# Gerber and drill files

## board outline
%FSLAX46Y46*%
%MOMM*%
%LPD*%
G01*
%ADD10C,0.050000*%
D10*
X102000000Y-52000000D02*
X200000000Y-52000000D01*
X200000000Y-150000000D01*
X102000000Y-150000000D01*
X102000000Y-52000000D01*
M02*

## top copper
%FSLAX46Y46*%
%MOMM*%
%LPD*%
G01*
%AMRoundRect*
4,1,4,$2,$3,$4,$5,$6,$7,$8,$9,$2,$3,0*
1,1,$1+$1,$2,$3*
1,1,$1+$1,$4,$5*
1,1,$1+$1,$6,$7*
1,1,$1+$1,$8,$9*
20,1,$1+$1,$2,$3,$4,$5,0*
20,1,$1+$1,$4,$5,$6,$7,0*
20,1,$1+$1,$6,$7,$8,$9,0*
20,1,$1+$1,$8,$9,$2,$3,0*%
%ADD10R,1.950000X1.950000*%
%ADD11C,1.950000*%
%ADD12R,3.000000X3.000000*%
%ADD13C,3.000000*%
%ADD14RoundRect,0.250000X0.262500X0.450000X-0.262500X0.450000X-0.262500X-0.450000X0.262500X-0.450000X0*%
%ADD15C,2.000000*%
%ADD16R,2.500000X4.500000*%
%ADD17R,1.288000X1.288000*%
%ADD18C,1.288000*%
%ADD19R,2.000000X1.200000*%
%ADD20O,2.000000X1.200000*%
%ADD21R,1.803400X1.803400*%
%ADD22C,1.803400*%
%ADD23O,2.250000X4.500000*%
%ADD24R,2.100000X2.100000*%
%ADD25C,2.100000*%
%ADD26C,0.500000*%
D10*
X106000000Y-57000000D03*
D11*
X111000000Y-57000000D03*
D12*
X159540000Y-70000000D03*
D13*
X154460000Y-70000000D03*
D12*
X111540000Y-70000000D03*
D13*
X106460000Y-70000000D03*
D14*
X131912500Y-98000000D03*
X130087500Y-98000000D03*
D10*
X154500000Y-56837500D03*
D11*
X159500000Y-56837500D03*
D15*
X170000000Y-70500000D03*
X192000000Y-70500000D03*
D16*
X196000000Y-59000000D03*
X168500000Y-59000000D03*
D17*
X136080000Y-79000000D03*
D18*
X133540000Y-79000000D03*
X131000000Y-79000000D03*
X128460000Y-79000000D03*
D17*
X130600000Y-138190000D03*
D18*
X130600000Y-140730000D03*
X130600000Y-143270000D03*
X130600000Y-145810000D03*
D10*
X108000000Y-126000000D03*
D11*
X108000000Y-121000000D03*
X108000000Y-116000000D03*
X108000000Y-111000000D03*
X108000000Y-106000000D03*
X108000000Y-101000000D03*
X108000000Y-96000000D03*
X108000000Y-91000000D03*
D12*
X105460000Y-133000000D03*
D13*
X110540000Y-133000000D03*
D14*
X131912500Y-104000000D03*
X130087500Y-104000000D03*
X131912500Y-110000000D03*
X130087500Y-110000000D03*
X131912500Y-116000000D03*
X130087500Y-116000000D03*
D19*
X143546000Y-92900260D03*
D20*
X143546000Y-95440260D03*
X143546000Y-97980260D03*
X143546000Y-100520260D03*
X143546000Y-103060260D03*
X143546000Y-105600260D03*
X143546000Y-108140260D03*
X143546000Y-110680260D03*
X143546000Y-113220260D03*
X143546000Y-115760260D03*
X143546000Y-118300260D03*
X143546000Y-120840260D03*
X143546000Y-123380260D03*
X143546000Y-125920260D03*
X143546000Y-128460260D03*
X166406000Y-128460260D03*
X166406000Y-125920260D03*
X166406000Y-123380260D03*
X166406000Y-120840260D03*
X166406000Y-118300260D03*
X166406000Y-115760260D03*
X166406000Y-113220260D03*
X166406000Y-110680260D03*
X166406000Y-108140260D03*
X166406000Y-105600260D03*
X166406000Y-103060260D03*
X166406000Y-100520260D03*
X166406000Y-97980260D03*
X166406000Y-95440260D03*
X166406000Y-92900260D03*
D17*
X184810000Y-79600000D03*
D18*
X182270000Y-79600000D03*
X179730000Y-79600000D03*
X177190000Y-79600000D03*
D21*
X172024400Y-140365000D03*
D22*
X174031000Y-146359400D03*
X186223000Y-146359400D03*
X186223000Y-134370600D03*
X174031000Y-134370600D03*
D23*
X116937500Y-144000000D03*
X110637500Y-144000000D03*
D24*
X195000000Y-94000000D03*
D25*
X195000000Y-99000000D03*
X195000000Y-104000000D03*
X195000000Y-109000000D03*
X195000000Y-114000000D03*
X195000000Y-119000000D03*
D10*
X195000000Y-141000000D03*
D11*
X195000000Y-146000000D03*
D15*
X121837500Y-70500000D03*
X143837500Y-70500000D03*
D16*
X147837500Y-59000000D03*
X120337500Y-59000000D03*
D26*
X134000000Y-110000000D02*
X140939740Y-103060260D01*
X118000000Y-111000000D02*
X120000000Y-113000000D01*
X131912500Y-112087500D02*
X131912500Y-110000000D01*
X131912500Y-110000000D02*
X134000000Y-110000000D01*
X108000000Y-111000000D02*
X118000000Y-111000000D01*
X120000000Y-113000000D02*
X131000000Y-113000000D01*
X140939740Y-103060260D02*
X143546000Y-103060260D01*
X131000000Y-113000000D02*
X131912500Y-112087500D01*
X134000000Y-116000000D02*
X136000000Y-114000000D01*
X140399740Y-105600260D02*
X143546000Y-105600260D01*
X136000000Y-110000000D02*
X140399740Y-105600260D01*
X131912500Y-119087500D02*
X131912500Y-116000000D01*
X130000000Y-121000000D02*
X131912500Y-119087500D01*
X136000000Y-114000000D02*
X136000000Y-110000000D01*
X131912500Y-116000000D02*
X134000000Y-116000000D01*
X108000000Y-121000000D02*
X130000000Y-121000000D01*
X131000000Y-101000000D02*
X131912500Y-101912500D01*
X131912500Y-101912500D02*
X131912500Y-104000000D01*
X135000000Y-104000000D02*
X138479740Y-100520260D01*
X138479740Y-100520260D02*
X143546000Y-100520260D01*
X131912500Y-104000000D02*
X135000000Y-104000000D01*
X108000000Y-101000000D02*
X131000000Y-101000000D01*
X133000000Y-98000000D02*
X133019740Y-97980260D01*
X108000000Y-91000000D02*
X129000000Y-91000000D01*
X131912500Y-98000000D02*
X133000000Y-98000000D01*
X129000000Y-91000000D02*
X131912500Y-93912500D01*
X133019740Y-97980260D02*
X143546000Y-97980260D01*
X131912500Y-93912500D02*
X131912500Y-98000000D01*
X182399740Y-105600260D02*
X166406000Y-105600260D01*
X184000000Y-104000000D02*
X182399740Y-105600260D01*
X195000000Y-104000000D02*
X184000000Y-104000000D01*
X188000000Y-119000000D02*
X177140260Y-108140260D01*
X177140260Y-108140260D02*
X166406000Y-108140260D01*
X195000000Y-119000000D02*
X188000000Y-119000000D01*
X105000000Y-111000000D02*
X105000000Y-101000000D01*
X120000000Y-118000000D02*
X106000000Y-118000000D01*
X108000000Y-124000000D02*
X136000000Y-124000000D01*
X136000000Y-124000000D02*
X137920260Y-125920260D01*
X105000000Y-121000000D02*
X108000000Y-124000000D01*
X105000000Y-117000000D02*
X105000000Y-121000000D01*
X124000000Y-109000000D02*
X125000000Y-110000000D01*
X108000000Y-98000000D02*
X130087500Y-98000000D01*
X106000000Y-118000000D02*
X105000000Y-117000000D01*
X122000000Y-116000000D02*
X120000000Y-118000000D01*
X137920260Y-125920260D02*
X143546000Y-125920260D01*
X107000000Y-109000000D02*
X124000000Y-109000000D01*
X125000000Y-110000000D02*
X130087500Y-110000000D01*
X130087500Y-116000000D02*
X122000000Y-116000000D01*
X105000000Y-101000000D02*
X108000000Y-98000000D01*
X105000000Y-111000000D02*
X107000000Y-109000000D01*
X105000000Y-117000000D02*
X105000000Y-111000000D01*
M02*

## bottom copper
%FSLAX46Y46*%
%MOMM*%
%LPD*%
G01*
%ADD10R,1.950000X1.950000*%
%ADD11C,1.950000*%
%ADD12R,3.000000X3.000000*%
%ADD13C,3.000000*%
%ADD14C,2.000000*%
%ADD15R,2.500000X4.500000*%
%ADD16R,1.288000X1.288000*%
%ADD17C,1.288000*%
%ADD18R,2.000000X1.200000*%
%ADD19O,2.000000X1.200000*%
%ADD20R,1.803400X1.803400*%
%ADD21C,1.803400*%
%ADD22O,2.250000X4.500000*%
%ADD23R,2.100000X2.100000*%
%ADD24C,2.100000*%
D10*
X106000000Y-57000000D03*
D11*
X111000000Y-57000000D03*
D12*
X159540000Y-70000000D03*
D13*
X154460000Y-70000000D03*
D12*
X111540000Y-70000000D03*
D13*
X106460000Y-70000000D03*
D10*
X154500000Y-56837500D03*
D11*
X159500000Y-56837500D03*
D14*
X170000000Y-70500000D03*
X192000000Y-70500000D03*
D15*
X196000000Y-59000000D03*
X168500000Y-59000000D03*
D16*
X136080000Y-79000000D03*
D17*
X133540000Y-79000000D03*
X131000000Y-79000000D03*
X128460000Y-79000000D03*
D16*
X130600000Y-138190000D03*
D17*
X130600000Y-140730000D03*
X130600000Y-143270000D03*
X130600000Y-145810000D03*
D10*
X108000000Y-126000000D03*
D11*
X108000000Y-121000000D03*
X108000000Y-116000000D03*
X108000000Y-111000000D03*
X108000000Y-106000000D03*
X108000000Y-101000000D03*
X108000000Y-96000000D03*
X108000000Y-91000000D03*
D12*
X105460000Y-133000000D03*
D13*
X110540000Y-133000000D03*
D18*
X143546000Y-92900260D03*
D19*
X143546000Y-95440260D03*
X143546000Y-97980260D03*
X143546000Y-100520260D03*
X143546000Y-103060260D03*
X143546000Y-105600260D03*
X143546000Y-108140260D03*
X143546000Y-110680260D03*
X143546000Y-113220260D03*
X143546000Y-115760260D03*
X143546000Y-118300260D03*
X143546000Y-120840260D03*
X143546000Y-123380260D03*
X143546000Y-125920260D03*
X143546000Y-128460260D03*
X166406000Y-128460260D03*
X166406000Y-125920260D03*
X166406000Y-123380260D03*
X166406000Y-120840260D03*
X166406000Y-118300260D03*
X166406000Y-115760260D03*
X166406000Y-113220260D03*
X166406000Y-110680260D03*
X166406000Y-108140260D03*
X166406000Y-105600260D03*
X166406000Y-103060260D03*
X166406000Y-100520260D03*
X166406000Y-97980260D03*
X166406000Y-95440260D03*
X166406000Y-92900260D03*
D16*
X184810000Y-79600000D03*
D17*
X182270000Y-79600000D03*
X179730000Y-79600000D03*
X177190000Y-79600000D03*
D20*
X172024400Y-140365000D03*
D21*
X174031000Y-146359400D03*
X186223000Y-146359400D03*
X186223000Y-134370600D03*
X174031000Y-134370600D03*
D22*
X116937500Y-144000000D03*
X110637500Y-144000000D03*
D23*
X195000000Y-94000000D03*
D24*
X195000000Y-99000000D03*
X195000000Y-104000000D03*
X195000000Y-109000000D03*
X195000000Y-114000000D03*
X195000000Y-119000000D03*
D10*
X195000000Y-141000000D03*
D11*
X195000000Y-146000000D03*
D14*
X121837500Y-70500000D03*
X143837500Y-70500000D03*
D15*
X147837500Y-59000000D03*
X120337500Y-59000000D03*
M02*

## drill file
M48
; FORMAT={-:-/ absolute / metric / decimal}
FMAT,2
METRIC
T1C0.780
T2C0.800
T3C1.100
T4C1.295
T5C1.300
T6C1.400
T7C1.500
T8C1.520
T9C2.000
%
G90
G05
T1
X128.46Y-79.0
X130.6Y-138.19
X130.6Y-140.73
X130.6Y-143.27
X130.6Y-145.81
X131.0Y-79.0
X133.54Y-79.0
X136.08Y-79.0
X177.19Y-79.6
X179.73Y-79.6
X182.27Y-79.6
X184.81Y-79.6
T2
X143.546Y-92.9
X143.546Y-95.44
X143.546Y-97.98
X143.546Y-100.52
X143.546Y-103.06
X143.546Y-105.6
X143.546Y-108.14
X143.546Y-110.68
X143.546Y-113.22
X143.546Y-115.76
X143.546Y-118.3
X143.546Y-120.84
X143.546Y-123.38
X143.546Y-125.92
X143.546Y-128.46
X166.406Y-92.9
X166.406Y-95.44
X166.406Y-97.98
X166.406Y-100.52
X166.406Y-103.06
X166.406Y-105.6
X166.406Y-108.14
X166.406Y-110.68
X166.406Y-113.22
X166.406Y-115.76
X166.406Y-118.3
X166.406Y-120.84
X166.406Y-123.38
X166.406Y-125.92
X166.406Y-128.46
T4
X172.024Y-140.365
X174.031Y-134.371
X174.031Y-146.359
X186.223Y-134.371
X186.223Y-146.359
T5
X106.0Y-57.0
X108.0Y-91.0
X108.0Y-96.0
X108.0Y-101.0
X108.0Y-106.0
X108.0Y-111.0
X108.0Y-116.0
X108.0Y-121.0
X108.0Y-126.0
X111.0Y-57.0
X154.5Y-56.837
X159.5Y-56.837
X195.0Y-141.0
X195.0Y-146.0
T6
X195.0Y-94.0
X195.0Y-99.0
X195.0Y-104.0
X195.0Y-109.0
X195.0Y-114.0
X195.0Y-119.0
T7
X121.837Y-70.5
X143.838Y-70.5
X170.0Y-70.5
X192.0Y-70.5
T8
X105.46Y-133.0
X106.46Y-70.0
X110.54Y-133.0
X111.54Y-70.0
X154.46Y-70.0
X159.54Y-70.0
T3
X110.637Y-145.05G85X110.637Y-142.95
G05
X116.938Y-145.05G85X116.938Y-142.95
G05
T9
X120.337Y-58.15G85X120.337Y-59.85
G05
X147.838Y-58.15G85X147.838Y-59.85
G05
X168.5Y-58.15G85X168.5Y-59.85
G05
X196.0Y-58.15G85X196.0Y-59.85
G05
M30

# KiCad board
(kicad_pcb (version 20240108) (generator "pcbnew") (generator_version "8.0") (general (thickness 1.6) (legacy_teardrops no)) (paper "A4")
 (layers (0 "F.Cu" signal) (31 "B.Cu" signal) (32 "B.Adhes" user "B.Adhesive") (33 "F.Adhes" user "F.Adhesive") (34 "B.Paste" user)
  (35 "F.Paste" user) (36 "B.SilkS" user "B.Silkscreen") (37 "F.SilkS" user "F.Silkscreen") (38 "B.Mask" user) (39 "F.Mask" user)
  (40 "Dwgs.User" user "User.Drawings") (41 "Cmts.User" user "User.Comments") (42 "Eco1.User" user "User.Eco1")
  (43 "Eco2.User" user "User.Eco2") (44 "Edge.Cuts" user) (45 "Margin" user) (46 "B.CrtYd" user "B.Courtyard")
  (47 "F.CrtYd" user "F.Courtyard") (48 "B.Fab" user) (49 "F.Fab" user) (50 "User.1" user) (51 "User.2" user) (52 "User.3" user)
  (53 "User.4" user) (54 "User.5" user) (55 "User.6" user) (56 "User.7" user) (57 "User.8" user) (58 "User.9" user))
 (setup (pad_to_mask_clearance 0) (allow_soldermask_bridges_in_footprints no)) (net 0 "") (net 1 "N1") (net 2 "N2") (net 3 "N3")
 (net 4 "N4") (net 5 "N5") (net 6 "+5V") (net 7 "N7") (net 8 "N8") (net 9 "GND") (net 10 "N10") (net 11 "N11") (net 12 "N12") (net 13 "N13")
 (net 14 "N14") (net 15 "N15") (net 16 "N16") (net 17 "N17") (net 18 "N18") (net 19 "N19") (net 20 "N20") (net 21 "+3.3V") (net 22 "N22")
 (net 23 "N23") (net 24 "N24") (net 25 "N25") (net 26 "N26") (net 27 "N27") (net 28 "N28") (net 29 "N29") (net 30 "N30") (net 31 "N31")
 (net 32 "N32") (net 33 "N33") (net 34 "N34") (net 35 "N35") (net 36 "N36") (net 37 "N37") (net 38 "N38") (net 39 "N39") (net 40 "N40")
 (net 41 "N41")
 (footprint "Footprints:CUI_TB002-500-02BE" (layer "F.Cu") (at 106 57)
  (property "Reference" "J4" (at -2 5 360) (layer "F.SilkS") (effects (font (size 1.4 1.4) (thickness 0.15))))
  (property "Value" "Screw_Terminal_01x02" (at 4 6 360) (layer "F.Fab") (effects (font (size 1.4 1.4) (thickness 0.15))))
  (pad "1" thru_hole rect (at 0 0) (size 1.95 1.95) (drill 1.3) (layers "*.Cu" "*.Mask") (remove_unused_layers no) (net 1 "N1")
   (solder_mask_margin 0.102))
  (pad "2" thru_hole circle (at 5 0) (size 1.95 1.95) (drill 1.3) (layers "*.Cu" "*.Mask") (remove_unused_layers no) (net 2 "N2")
   (solder_mask_margin 0.102)))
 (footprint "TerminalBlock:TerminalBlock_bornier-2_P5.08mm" (layer "F.Cu") (at 159.54 70 180)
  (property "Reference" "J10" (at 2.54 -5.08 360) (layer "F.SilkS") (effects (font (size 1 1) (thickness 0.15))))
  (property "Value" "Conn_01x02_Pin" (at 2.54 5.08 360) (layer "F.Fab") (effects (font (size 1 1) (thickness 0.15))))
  (pad "1" thru_hole rect (at 0 0 180) (size 3 3) (drill 1.52) (layers "*.Cu" "*.Mask") (remove_unused_layers no) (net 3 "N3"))
  (pad "2" thru_hole circle (at 5.08 0 180) (size 3 3) (drill 1.52) (layers "*.Cu" "*.Mask") (remove_unused_layers no) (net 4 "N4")))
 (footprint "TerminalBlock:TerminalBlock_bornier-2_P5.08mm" (layer "F.Cu") (at 111.54 70 180)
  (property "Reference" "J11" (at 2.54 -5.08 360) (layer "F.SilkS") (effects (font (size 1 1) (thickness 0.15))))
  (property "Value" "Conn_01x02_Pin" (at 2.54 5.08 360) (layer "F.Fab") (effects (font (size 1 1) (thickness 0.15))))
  (pad "1" thru_hole rect (at 0 0 180) (size 3 3) (drill 1.52) (layers "*.Cu" "*.Mask") (remove_unused_layers no) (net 2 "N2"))
  (pad "2" thru_hole circle (at 5.08 0 180) (size 3 3) (drill 1.52) (layers "*.Cu" "*.Mask") (remove_unused_layers no) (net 1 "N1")))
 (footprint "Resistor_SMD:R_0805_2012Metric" (layer "F.Cu") (at 131 98 180)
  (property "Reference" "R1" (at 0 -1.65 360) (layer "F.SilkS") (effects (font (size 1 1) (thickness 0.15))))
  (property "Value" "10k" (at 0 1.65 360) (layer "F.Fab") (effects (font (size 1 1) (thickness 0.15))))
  (pad "1" smd roundrect (at -0.9125 0 180) (size 1.025 1.4) (layers "F.Cu" "F.Paste" "F.Mask") (roundrect_rratio 0.243902) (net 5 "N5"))
  (pad "2" smd roundrect (at 0.9125 0 180) (size 1.025 1.4) (layers "F.Cu" "F.Paste" "F.Mask") (roundrect_rratio 0.243902) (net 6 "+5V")))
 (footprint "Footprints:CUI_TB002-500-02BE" (layer "F.Cu") (at 154.5 56.8375)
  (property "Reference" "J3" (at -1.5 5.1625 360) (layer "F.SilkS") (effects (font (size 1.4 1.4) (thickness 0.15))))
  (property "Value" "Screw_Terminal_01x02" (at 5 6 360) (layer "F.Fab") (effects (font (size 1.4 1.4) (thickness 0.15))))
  (pad "1" thru_hole rect (at 0 0) (size 1.95 1.95) (drill 1.3) (layers "*.Cu" "*.Mask") (remove_unused_layers no) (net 4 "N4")
   (solder_mask_margin 0.102))
  (pad "2" thru_hole circle (at 5 0) (size 1.95 1.95) (drill 1.3) (layers "*.Cu" "*.Mask") (remove_unused_layers no) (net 3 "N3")
   (solder_mask_margin 0.102)))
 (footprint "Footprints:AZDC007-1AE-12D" (layer "F.Cu") (at 181 64)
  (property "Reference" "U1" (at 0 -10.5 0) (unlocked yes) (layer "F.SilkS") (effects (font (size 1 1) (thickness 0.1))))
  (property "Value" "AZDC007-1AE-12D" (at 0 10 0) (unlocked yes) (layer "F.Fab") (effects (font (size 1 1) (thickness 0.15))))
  (pad "1" thru_hole circle (at -11 6.5) (size 2 2) (drill 1.5) (layers "*.Cu" "*.Mask") (remove_unused_layers no) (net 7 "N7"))
  (pad "2" thru_hole circle (at 11 6.5) (size 2 2) (drill 1.5) (layers "*.Cu" "*.Mask") (remove_unused_layers no) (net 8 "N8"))
  (pad "3" thru_hole rect (at 15 -5) (size 2.5 4.5) (drill oval 2 3.7) (layers "*.Cu" "*.Mask") (remove_unused_layers no) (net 3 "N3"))
  (pad "4" thru_hole rect (at -12.5 -5) (size 2.5 4.5) (drill oval 2 3.7) (layers "*.Cu" "*.Mask") (remove_unused_layers no) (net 4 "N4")))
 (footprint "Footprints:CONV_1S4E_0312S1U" (layer "F.Cu") (at 132.27 80.4 180)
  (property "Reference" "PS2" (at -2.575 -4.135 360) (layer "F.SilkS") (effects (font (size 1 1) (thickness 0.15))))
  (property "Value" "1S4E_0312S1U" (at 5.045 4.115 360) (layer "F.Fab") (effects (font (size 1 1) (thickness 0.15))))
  (pad "1" thru_hole rect (at -3.81 1.4 180) (size 1.288 1.288) (drill 0.78) (layers "*.Cu" "*.Mask") (remove_unused_layers no)
   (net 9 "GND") (solder_mask_margin 0.102))
  (pad "2" thru_hole circle (at -1.27 1.4 180) (size 1.288 1.288) (drill 0.78) (layers "*.Cu" "*.Mask") (remove_unused_layers no)
   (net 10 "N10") (solder_mask_margin 0.102))
  (pad "3" thru_hole circle (at 1.27 1.4 180) (size 1.288 1.288) (drill 0.78) (layers "*.Cu" "*.Mask") (remove_unused_layers no)
   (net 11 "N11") (solder_mask_margin 0.102))
  (pad "4" thru_hole circle (at 3.81 1.4 180) (size 1.288 1.288) (drill 0.78) (layers "*.Cu" "*.Mask") (remove_unused_layers no)
   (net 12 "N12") (solder_mask_margin 0.102)))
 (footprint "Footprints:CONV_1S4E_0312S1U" (layer "F.Cu") (at 132 142 -90)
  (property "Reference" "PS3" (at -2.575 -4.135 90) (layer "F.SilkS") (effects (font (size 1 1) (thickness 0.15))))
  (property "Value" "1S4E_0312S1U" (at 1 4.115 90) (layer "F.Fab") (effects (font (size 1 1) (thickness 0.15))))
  (pad "1" thru_hole rect (at -3.81 1.4 270) (size 1.288 1.288) (drill 0.78) (layers "*.Cu" "*.Mask") (remove_unused_layers no)
   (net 9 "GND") (solder_mask_margin 0.102))
  (pad "2" thru_hole circle (at -1.27 1.4 270) (size 1.288 1.288) (drill 0.78) (layers "*.Cu" "*.Mask") (remove_unused_layers no)
   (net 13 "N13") (solder_mask_margin 0.102))
  (pad "3" thru_hole circle (at 1.27 1.4 270) (size 1.288 1.288) (drill 0.78) (layers "*.Cu" "*.Mask") (remove_unused_layers no)
   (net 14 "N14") (solder_mask_margin 0.102))
  (pad "4" thru_hole circle (at 3.81 1.4 270) (size 1.288 1.288) (drill 0.78) (layers "*.Cu" "*.Mask") (remove_unused_layers no)
   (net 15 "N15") (solder_mask_margin 0.102)))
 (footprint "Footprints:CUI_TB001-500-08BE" (layer "F.Cu") (at 108 126 90)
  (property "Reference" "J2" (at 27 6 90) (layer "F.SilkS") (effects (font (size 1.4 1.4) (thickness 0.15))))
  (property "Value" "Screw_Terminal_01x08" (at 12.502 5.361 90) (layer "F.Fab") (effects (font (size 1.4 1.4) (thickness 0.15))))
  (pad "1" thru_hole rect (at 0 0 90) (size 1.95 1.95) (drill 1.3) (layers "*.Cu" "*.Mask") (remove_unused_layers no) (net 9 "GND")
   (solder_mask_margin 0.102))
  (pad "2" thru_hole circle (at 5 0 90) (size 1.95 1.95) (drill 1.3) (layers "*.Cu" "*.Mask") (remove_unused_layers no) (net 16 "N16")
   (solder_mask_margin 0.102))
  (pad "3" thru_hole circle (at 10 0 90) (size 1.95 1.95) (drill 1.3) (layers "*.Cu" "*.Mask") (remove_unused_layers no) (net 9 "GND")
   (solder_mask_margin 0.102))
  (pad "4" thru_hole circle (at 15 0 90) (size 1.95 1.95) (drill 1.3) (layers "*.Cu" "*.Mask") (remove_unused_layers no) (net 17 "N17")
   (solder_mask_margin 0.102))
  (pad "5" thru_hole circle (at 20 0 90) (size 1.95 1.95) (drill 1.3) (layers "*.Cu" "*.Mask") (remove_unused_layers no) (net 9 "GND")
   (solder_mask_margin 0.102))
  (pad "6" thru_hole circle (at 25 0 90) (size 1.95 1.95) (drill 1.3) (layers "*.Cu" "*.Mask") (remove_unused_layers no) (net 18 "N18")
   (solder_mask_margin 0.102))
  (pad "7" thru_hole circle (at 30 0 90) (size 1.95 1.95) (drill 1.3) (layers "*.Cu" "*.Mask") (remove_unused_layers no) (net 9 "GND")
   (solder_mask_margin 0.102))
  (pad "8" thru_hole circle (at 35 0 90) (size 1.95 1.95) (drill 1.3) (layers "*.Cu" "*.Mask") (remove_unused_layers no) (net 5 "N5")
   (solder_mask_margin 0.102)))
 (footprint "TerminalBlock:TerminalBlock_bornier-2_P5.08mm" (layer "F.Cu") (at 105.46 133)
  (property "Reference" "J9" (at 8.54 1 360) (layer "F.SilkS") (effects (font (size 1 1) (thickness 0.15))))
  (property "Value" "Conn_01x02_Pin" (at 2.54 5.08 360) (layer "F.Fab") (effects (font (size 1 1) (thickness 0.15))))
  (pad "1" thru_hole rect (at 0 0) (size 3 3) (drill 1.52) (layers "*.Cu" "*.Mask") (remove_unused_layers no) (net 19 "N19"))
  (pad "2" thru_hole circle (at 5.08 0) (size 3 3) (drill 1.52) (layers "*.Cu" "*.Mask") (remove_unused_layers no) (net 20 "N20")))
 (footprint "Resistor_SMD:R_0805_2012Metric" (layer "F.Cu") (at 131 104 180)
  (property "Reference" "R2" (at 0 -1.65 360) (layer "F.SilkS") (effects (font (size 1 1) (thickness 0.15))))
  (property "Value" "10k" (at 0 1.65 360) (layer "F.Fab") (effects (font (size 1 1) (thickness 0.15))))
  (pad "1" smd roundrect (at -0.9125 0 180) (size 1.025 1.4) (layers "F.Cu" "F.Paste" "F.Mask") (roundrect_rratio 0.243902) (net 18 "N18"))
  (pad "2" smd roundrect (at 0.9125 0 180) (size 1.025 1.4) (layers "F.Cu" "F.Paste" "F.Mask") (roundrect_rratio 0.243902) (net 6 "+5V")))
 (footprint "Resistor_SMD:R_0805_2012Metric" (layer "F.Cu") (at 131 110 180)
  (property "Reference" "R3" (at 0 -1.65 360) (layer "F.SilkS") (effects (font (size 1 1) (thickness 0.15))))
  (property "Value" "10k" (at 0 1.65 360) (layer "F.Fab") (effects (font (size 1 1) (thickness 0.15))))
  (pad "1" smd roundrect (at -0.9125 0 180) (size 1.025 1.4) (layers "F.Cu" "F.Paste" "F.Mask") (roundrect_rratio 0.243902) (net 17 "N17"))
  (pad "2" smd roundrect (at 0.9125 0 180) (size 1.025 1.4) (layers "F.Cu" "F.Paste" "F.Mask") (roundrect_rratio 0.243902) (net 6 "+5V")))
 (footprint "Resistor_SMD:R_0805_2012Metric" (layer "F.Cu") (at 131 116 180)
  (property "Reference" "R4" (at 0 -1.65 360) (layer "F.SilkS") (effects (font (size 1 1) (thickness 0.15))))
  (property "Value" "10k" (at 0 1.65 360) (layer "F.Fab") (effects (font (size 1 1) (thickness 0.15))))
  (pad "1" smd roundrect (at -0.9125 0 180) (size 1.025 1.4) (layers "F.Cu" "F.Paste" "F.Mask") (roundrect_rratio 0.243902) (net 16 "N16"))
  (pad "2" smd roundrect (at 0.9125 0 180) (size 1.025 1.4) (layers "F.Cu" "F.Paste" "F.Mask") (roundrect_rratio 0.243902) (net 6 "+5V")))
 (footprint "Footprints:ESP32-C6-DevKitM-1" (layer "F.Cu") (at 143.546 92.90026)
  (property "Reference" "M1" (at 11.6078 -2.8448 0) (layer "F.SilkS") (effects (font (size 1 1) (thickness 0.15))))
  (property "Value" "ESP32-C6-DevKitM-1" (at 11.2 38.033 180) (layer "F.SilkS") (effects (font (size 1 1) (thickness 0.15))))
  (pad "1" thru_hole rect (at 0 0 270) (size 1.2 2) (drill 0.8) (layers "*.Cu" "*.Mask") (remove_unused_layers no) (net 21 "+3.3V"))
  (pad "2" thru_hole oval (at 0 2.54 270) (size 1.2 2) (drill 0.8) (layers "*.Cu" "*.Mask") (remove_unused_layers no) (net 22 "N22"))
  (pad "3" thru_hole oval (at 0 5.08 270) (size 1.2 2) (drill 0.8) (layers "*.Cu" "*.Mask") (remove_unused_layers no) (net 5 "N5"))
  (pad "4" thru_hole oval (at 0 7.62 270) (size 1.2 2) (drill 0.8) (layers "*.Cu" "*.Mask") (remove_unused_layers no) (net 18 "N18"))
  (pad "5" thru_hole oval (at 0 10.16 270) (size 1.2 2) (drill 0.8) (layers "*.Cu" "*.Mask") (remove_unused_layers no) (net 17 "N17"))
  (pad "6" thru_hole oval (at 0 12.7 270) (size 1.2 2) (drill 0.8) (layers "*.Cu" "*.Mask") (remove_unused_layers no) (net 16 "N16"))
  (pad "7" thru_hole oval (at 0 15.24 270) (size 1.2 2) (drill 0.8) (layers "*.Cu" "*.Mask") (remove_unused_layers no) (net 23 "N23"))
  (pad "8" thru_hole oval (at 0 17.78 270) (size 1.2 2) (drill 0.8) (layers "*.Cu" "*.Mask") (remove_unused_layers no) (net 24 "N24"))
  (pad "9" thru_hole oval (at 0 20.32 270) (size 1.2 2) (drill 0.8) (layers "*.Cu" "*.Mask") (remove_unused_layers no) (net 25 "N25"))
  (pad "10" thru_hole oval (at 0 22.86 270) (size 1.2 2) (drill 0.8) (layers "*.Cu" "*.Mask") (remove_unused_layers no) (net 13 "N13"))
  (pad "11" thru_hole oval (at 0 25.4 270) (size 1.2 2) (drill 0.8) (layers "*.Cu" "*.Mask") (remove_unused_layers no) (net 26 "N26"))
  (pad "12" thru_hole oval (at 0 27.94 270) (size 1.2 2) (drill 0.8) (layers "*.Cu" "*.Mask") (remove_unused_layers no) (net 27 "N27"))
  (pad "13" thru_hole oval (at 0 30.48 270) (size 1.2 2) (drill 0.8) (layers "*.Cu" "*.Mask") (remove_unused_layers no) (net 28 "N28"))
  (pad "14" thru_hole oval (at 0 33.02 270) (size 1.2 2) (drill 0.8) (layers "*.Cu" "*.Mask") (remove_unused_layers no) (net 6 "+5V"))
  (pad "15" thru_hole oval (at 0 35.56 270) (size 1.2 2) (drill 0.8) (layers "*.Cu" "*.Mask") (remove_unused_layers no) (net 9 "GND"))
  (pad "16" thru_hole oval (at 22.86 35.56 270) (size 1.2 2) (drill 0.8) (layers "*.Cu" "*.Mask") (remove_unused_layers no) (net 9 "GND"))
  (pad "17" thru_hole oval (at 22.86 33.02 270) (size 1.2 2) (drill 0.8) (layers "*.Cu" "*.Mask") (remove_unused_layers no) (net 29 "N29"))
  (pad "18" thru_hole oval (at 22.86 30.48 270) (size 1.2 2) (drill 0.8) (layers "*.Cu" "*.Mask") (remove_unused_layers no) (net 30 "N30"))
  (pad "19" thru_hole oval (at 22.86 27.94 270) (size 1.2 2) (drill 0.8) (layers "*.Cu" "*.Mask") (remove_unused_layers no) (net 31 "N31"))
  (pad "20" thru_hole oval (at 22.86 25.4 270) (size 1.2 2) (drill 0.8) (layers "*.Cu" "*.Mask") (remove_unused_layers no) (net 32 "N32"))
  (pad "21" thru_hole oval (at 22.86 22.86 270) (size 1.2 2) (drill 0.8) (layers "*.Cu" "*.Mask") (remove_unused_layers no) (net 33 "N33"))
  (pad "22" thru_hole oval (at 22.86 20.32 270) (size 1.2 2) (drill 0.8) (layers "*.Cu" "*.Mask") (remove_unused_layers no) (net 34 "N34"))
  (pad "23" thru_hole oval (at 22.86 17.78 270) (size 1.2 2) (drill 0.8) (layers "*.Cu" "*.Mask") (remove_unused_layers no) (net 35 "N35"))
  (pad "24" thru_hole oval (at 22.86 15.24 270) (size 1.2 2) (drill 0.8) (layers "*.Cu" "*.Mask") (remove_unused_layers no) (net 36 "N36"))
  (pad "25" thru_hole oval (at 22.86 12.7 270) (size 1.2 2) (drill 0.8) (layers "*.Cu" "*.Mask") (remove_unused_layers no) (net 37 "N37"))
  (pad "26" thru_hole oval (at 22.86 10.16 270) (size 1.2 2) (drill 0.8) (layers "*.Cu" "*.Mask") (remove_unused_layers no) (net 10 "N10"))
  (pad "27" thru_hole oval (at 22.86 7.62 270) (size 1.2 2) (drill 0.8) (layers "*.Cu" "*.Mask") (remove_unused_layers no) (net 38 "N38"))
  (pad "28" thru_hole oval (at 22.86 5.08 270) (size 1.2 2) (drill 0.8) (layers "*.Cu" "*.Mask") (remove_unused_layers no) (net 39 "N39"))
  (pad "29" thru_hole oval (at 22.86 2.54 270) (size 1.2 2) (drill 0.8) (layers "*.Cu" "*.Mask") (remove_unused_layers no) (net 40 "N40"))
  (pad "30" thru_hole oval (at 22.86 0 270) (size 1.2 2) (drill 0.8) (layers "*.Cu" "*.Mask") (remove_unused_layers no) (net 9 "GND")))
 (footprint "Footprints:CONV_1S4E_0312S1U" (layer "F.Cu") (at 181 81 180)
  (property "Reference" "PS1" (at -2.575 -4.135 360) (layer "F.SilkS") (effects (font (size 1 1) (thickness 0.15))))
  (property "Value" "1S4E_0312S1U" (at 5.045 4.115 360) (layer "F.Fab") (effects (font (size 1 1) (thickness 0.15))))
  (pad "1" thru_hole rect (at -3.81 1.4 180) (size 1.288 1.288) (drill 0.78) (layers "*.Cu" "*.Mask") (remove_unused_layers no)
   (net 9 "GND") (solder_mask_margin 0.102))
  (pad "2" thru_hole circle (at -1.27 1.4 180) (size 1.288 1.288) (drill 0.78) (layers "*.Cu" "*.Mask") (remove_unused_layers no)
   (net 38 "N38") (solder_mask_margin 0.102))
  (pad "3" thru_hole circle (at 1.27 1.4 180) (size 1.288 1.288) (drill 0.78) (layers "*.Cu" "*.Mask") (remove_unused_layers no)
   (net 8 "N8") (solder_mask_margin 0.102))
  (pad "4" thru_hole circle (at 3.81 1.4 180) (size 1.288 1.288) (drill 0.78) (layers "*.Cu" "*.Mask") (remove_unused_layers no)
   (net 7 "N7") (solder_mask_margin 0.102)))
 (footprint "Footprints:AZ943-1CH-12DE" (layer "F.Cu") (at 172.0244 140.365 90)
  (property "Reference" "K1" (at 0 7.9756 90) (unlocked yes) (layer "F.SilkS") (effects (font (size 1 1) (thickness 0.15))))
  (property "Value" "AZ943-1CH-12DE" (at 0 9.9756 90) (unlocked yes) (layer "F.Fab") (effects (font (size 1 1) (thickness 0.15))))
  (pad "1" thru_hole rect (at 0 0 90) (size 1.8034 1.8034) (drill 1.2954) (layers "*.Cu" "*.Mask") (remove_unused_layers no) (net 19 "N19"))
  (pad "2" thru_hole circle (at -5.9944 2.0066 90) (size 1.8034 1.8034) (drill 1.2954) (layers "*.Cu" "*.Mask") (remove_unused_layers no)
   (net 15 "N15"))
  (pad "3" thru_hole circle (at -5.9944 14.1986 90) (size 1.8034 1.8034) (drill 1.2954) (layers "*.Cu" "*.Mask") (remove_unused_layers no)
   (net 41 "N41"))
  (pad "4" thru_hole circle (at 5.9944 14.1986 90) (size 1.8034 1.8034) (drill 1.2954) (layers "*.Cu" "*.Mask") (remove_unused_layers no)
   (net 19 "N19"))
  (pad "5" thru_hole circle (at 5.9944 2.0066 90) (size 1.8034 1.8034) (drill 1.2954) (layers "*.Cu" "*.Mask") (remove_unused_layers no)
   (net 14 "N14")))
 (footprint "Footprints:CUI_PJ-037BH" (layer "F.Cu") (at 116.9375 144 180)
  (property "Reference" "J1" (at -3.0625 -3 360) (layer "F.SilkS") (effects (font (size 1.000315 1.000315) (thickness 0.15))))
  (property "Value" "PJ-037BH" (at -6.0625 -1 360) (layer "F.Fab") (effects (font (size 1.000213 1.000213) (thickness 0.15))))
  (pad "1" thru_hole oval (at 0 0 180) (size 2.25 4.5) (drill oval 1.1 3.2) (layers "*.Cu" "*.Mask") (remove_unused_layers no)
   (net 20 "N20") (solder_mask_margin 0.102))
  (pad "2" thru_hole oval (at 6.3 0 180) (size 2.25 4.5) (drill oval 1.1 3.2) (layers "*.Cu" "*.Mask") (remove_unused_layers no)
   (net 19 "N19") (solder_mask_margin 0.102)))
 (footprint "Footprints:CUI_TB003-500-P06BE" (layer "F.Cu") (at 195 94 -90)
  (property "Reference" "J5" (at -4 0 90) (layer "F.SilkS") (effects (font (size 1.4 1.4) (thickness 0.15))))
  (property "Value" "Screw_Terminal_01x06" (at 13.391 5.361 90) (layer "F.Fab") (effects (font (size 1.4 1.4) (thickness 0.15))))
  (pad "1" thru_hole rect (at 0 0 270) (size 2.1 2.1) (drill 1.4) (layers "*.Cu" "*.Mask") (remove_unused_layers no) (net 21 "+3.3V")
   (solder_mask_margin 0.102))
  (pad "2" thru_hole circle (at 5 0 270) (size 2.1 2.1) (drill 1.4) (layers "*.Cu" "*.Mask") (remove_unused_layers no) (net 9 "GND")
   (solder_mask_margin 0.102))
  (pad "3" thru_hole circle (at 10 0 270) (size 2.1 2.1) (drill 1.4) (layers "*.Cu" "*.Mask") (remove_unused_layers no) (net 37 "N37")
   (solder_mask_margin 0.102))
  (pad "4" thru_hole circle (at 15 0 270) (size 2.1 2.1) (drill 1.4) (layers "*.Cu" "*.Mask") (remove_unused_layers no) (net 21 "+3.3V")
   (solder_mask_margin 0.102))
  (pad "5" thru_hole circle (at 20 0 270) (size 2.1 2.1) (drill 1.4) (layers "*.Cu" "*.Mask") (remove_unused_layers no) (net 9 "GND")
   (solder_mask_margin 0.102))
  (pad "6" thru_hole circle (at 25 0 270) (size 2.1 2.1) (drill 1.4) (layers "*.Cu" "*.Mask") (remove_unused_layers no) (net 36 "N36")
   (solder_mask_margin 0.102)))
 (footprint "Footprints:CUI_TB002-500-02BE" (layer "F.Cu") (at 195 141 -90)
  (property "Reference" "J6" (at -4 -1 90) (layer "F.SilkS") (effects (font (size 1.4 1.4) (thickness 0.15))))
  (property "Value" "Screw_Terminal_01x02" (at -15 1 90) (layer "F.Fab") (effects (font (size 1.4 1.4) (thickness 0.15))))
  (pad "1" thru_hole rect (at 0 0 270) (size 1.95 1.95) (drill 1.3) (layers "*.Cu" "*.Mask") (remove_unused_layers no) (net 20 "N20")
   (solder_mask_margin 0.102))
  (pad "2" thru_hole circle (at 5 0 270) (size 1.95 1.95) (drill 1.3) (layers "*.Cu" "*.Mask") (remove_unused_layers no) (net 41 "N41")
   (solder_mask_margin 0.102)))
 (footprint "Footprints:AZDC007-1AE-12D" (layer "F.Cu") (at 132.8375 64)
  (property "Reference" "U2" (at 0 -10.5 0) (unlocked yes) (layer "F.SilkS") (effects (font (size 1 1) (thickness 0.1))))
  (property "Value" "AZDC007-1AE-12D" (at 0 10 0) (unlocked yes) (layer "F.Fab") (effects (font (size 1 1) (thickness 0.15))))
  (pad "1" thru_hole circle (at -11 6.5) (size 2 2) (drill 1.5) (layers "*.Cu" "*.Mask") (remove_unused_layers no) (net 12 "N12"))
  (pad "2" thru_hole circle (at 11 6.5) (size 2 2) (drill 1.5) (layers "*.Cu" "*.Mask") (remove_unused_layers no) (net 11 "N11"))
  (pad "3" thru_hole rect (at 15 -5) (size 2.5 4.5) (drill oval 2 3.7) (layers "*.Cu" "*.Mask") (remove_unused_layers no) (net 2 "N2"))
  (pad "4" thru_hole rect (at -12.5 -5) (size 2.5 4.5) (drill oval 2 3.7) (layers "*.Cu" "*.Mask") (remove_unused_layers no) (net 1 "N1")))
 (gr_rect (start 102 52) (end 200 150) (stroke (width 0.05) (type default)) (fill none) (layer "Edge.Cuts"))
 (segment (start 134 110) (end 140.93974 103.06026) (width 0.5) (layer "F.Cu") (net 17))
 (segment (start 118 111) (end 120 113) (width 0.5) (layer "F.Cu") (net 17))
 (segment (start 131.9125 112.0875) (end 131.9125 110) (width 0.5) (layer "F.Cu") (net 17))
 (segment (start 131.9125 110) (end 134 110) (width 0.5) (layer "F.Cu") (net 17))
 (segment (start 108 111) (end 118 111) (width 0.5) (layer "F.Cu") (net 17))
 (segment (start 120 113) (end 131 113) (width 0.5) (layer "F.Cu") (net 17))
 (segment (start 140.93974 103.06026) (end 143.546 103.06026) (width 0.5) (layer "F.Cu") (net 17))
 (segment (start 131 113) (end 131.9125 112.0875) (width 0.5) (layer "F.Cu") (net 17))
 (segment (start 134 116) (end 136 114) (width 0.5) (layer "F.Cu") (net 16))
 (segment (start 140.39974 105.60026) (end 143.546 105.60026) (width 0.5) (layer "F.Cu") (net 16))
 (segment (start 136 110) (end 140.39974 105.60026) (width 0.5) (layer "F.Cu") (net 16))
 (segment (start 131.9125 119.0875) (end 131.9125 116) (width 0.5) (layer "F.Cu") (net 16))
 (segment (start 130 121) (end 131.9125 119.0875) (width 0.5) (layer "F.Cu") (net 16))
 (segment (start 136 114) (end 136 110) (width 0.5) (layer "F.Cu") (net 16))
 (segment (start 131.9125 116) (end 134 116) (width 0.5) (layer "F.Cu") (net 16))
 (segment (start 108 121) (end 130 121) (width 0.5) (layer "F.Cu") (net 16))
 (segment (start 131 101) (end 131.9125 101.9125) (width 0.5) (layer "F.Cu") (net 18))
 (segment (start 131.9125 101.9125) (end 131.9125 104) (width 0.5) (layer "F.Cu") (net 18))
 (segment (start 135 104) (end 138.47974 100.52026) (width 0.5) (layer "F.Cu") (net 18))
 (segment (start 138.47974 100.52026) (end 143.546 100.52026) (width 0.5) (layer "F.Cu") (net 18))
 (segment (start 131.9125 104) (end 135 104) (width 0.5) (layer "F.Cu") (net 18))
 (segment (start 108 101) (end 131 101) (width 0.5) (layer "F.Cu") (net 18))
 (segment (start 133 98) (end 133.01974 97.98026) (width 0.5) (layer "F.Cu") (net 5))
 (segment (start 108 91) (end 129 91) (width 0.5) (layer "F.Cu") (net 5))
 (segment (start 131.9125 98) (end 133 98) (width 0.5) (layer "F.Cu") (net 5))
 (segment (start 129 91) (end 131.9125 93.9125) (width 0.5) (layer "F.Cu") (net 5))
 (segment (start 133.01974 97.98026) (end 143.546 97.98026) (width 0.5) (layer "F.Cu") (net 5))
 (segment (start 131.9125 93.9125) (end 131.9125 98) (width 0.5) (layer "F.Cu") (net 5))
 (segment (start 182.39974 105.60026) (end 166.406 105.60026) (width 0.5) (layer "F.Cu") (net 37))
 (segment (start 184 104) (end 182.39974 105.60026) (width 0.5) (layer "F.Cu") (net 37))
 (segment (start 195 104) (end 184 104) (width 0.5) (layer "F.Cu") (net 37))
 (segment (start 188 119) (end 177.14026 108.14026) (width 0.5) (layer "F.Cu") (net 36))
 (segment (start 177.14026 108.14026) (end 166.406 108.14026) (width 0.5) (layer "F.Cu") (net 36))
 (segment (start 195 119) (end 188 119) (width 0.5) (layer "F.Cu") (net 36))
 (segment (start 105 111) (end 105 101) (width 0.5) (layer "F.Cu") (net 6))
 (segment (start 120 118) (end 106 118) (width 0.5) (layer "F.Cu") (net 6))
 (segment (start 108 124) (end 136 124) (width 0.5) (layer "F.Cu") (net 6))
 (segment (start 136 124) (end 137.92026 125.92026) (width 0.5) (layer "F.Cu") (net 6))
 (segment (start 105 121) (end 108 124) (width 0.5) (layer "F.Cu") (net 6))
 (segment (start 105 117) (end 105 121) (width 0.5) (layer "F.Cu") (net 6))
 (segment (start 124 109) (end 125 110) (width 0.5) (layer "F.Cu") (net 6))
 (segment (start 108 98) (end 130.0875 98) (width 0.5) (layer "F.Cu") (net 6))
 (segment (start 106 118) (end 105 117) (width 0.5) (layer "F.Cu") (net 6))
 (segment (start 122 116) (end 120 118) (width 0.5) (layer "F.Cu") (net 6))
 (segment (start 137.92026 125.92026) (end 143.546 125.92026) (width 0.5) (layer "F.Cu") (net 6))
 (segment (start 107 109) (end 124 109) (width 0.5) (layer "F.Cu") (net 6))
 (segment (start 125 110) (end 130.0875 110) (width 0.5) (layer "F.Cu") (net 6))
 (segment (start 130.0875 116) (end 122 116) (width 0.5) (layer "F.Cu") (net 6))
 (segment (start 105 101) (end 108 98) (width 0.5) (layer "F.Cu") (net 6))
 (segment (start 105 111) (end 107 109) (width 0.5) (layer "F.Cu") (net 6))
 (segment (start 105 117) (end 105 111) (width 0.5) (layer "F.Cu") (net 6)))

